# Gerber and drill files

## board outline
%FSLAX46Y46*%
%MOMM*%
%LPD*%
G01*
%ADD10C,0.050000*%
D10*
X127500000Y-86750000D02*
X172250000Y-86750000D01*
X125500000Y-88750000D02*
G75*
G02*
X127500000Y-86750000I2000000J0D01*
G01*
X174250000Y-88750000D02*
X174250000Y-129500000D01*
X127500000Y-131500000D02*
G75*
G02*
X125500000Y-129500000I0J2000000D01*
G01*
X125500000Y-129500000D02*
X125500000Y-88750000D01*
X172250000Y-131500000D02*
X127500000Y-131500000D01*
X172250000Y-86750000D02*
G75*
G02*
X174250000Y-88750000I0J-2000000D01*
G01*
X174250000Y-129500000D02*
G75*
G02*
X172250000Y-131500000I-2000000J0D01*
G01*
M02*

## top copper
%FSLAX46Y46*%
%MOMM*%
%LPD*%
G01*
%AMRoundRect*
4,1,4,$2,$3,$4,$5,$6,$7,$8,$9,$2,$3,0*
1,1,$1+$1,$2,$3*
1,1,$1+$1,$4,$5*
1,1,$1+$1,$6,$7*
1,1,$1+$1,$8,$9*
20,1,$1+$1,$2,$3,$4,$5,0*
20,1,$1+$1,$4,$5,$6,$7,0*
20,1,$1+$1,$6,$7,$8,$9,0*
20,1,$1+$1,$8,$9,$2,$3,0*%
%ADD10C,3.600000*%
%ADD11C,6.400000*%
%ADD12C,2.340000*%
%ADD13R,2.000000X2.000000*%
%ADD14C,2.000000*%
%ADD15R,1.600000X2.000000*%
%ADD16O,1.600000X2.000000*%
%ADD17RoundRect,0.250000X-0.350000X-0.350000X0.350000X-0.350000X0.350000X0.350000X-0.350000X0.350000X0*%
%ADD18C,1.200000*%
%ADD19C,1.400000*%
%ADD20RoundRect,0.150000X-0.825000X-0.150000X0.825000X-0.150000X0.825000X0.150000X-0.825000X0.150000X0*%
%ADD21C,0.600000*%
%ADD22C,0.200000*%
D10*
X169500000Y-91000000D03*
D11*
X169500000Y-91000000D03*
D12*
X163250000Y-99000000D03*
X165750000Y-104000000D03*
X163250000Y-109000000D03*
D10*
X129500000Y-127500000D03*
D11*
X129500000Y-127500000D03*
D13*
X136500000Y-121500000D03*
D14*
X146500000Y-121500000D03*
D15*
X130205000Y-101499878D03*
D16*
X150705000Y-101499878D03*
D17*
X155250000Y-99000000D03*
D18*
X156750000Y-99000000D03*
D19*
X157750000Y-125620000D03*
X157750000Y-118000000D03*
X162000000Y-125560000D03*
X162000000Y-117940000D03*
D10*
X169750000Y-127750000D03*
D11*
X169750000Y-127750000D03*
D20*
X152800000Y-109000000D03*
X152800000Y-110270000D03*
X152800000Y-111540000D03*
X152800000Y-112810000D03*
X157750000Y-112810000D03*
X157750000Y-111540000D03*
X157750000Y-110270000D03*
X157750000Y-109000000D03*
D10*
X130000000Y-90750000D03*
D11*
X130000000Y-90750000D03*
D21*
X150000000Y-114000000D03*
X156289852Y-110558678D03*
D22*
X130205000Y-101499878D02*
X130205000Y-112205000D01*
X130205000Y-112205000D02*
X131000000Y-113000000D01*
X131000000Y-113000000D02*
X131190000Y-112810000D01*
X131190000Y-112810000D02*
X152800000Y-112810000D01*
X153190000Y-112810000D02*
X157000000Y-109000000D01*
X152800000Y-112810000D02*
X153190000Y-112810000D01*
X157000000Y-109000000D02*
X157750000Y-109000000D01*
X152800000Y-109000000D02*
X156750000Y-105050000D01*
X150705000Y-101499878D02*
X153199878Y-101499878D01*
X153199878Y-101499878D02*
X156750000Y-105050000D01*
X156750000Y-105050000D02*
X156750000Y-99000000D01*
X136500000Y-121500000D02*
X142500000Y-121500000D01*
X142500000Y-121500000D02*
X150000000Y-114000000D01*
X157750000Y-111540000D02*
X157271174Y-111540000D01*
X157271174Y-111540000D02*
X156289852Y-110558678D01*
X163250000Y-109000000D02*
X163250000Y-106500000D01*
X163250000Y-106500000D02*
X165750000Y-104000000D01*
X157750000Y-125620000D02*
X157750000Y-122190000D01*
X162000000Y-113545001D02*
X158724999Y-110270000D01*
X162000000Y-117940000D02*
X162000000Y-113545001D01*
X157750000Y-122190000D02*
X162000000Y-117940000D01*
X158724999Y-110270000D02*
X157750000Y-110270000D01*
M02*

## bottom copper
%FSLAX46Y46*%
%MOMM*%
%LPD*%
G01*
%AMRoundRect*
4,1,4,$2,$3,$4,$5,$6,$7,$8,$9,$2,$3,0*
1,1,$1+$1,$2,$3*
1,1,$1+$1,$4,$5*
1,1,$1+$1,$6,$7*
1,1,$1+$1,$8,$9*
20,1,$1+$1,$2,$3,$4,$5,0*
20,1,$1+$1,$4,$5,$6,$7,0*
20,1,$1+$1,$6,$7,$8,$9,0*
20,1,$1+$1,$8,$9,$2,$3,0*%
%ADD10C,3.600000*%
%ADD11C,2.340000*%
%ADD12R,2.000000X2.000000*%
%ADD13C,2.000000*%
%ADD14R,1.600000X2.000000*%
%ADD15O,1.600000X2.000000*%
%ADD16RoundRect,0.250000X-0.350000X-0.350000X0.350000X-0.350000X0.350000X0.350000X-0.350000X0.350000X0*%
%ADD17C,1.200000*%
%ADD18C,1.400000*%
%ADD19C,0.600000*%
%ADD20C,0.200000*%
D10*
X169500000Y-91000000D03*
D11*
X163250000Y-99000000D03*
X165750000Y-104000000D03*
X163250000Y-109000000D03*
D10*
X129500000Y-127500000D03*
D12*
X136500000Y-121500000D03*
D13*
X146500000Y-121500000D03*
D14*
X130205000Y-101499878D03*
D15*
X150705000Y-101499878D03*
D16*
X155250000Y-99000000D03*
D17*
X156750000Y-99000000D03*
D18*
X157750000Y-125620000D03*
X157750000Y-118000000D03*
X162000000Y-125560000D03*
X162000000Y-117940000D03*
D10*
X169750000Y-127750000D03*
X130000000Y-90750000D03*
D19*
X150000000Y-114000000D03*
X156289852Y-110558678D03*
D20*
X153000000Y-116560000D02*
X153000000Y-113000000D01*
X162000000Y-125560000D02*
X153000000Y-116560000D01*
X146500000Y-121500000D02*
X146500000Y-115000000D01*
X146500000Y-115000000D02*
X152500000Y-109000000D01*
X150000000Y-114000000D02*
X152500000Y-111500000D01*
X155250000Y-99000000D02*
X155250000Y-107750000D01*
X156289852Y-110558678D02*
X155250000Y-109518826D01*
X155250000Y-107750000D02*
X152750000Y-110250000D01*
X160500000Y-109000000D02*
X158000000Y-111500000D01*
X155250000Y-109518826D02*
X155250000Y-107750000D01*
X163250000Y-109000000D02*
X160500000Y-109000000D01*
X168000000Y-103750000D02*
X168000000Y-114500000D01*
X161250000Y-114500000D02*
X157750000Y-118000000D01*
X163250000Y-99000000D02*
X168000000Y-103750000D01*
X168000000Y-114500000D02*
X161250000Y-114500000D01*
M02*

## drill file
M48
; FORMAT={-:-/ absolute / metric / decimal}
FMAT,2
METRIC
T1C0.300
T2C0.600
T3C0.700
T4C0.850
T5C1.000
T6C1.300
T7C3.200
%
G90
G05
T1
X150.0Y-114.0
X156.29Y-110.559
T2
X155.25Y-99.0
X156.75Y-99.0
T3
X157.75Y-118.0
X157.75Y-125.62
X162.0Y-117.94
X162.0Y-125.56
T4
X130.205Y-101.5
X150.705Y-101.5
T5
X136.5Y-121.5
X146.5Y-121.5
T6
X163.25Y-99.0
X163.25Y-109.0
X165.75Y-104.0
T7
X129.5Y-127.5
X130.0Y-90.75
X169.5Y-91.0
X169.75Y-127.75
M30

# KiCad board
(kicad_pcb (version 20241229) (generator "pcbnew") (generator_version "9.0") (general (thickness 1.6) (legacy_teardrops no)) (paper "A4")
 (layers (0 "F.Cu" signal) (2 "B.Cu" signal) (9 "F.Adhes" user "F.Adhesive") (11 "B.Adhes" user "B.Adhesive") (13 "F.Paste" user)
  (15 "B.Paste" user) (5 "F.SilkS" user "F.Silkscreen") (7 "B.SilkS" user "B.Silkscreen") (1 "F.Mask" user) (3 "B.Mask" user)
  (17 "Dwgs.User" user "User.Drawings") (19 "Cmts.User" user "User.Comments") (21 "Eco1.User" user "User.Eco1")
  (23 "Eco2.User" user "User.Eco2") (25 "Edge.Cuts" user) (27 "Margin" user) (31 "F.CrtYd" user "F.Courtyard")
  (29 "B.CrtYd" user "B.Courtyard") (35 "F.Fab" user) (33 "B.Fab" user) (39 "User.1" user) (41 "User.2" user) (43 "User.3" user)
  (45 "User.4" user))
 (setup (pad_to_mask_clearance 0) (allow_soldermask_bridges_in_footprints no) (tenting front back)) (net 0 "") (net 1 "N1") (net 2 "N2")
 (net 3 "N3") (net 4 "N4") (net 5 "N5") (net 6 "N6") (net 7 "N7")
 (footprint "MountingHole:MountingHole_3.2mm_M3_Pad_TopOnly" (layer "F.Cu") (at 169.5 91)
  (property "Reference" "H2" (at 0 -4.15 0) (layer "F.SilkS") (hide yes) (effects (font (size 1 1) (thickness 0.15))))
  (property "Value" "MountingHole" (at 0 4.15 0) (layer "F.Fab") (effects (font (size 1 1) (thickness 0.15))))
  (pad "1" thru_hole circle (at 0 0) (size 3.6 3.6) (drill 3.2) (layers "*.Cu" "*.Mask") (remove_unused_layers no) (zone_connect 2))
  (pad "1" connect circle (at 0 0) (size 6.4 6.4) (layers "F.Cu" "F.Mask") (zone_connect 2)))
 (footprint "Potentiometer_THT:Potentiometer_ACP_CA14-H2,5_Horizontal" (layer "F.Cu") (at 163.25 99)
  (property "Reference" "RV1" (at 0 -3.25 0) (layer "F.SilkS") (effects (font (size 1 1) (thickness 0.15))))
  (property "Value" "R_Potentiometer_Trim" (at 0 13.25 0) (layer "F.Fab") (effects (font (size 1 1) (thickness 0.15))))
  (pad "1" thru_hole circle (at 0 0) (size 2.34 2.34) (drill 1.3) (layers "*.Cu" "*.Mask") (remove_unused_layers no) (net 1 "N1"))
  (pad "2" thru_hole circle (at 2.5 5) (size 2.34 2.34) (drill 1.3) (layers "*.Cu" "*.Mask") (remove_unused_layers no) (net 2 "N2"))
  (pad "3" thru_hole circle (at 0 10) (size 2.34 2.34) (drill 1.3) (layers "*.Cu" "*.Mask") (remove_unused_layers no) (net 2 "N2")))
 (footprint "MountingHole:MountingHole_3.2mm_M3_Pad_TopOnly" (layer "F.Cu") (at 129.5 127.5)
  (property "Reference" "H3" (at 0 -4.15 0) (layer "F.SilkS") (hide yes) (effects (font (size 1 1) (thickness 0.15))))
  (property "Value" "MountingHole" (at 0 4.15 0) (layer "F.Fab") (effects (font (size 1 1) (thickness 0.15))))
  (pad "1" thru_hole circle (at 0 0) (size 3.6 3.6) (drill 3.2) (layers "*.Cu" "*.Mask") (remove_unused_layers no) (zone_connect 2))
  (pad "1" connect circle (at 0 0) (size 6.4 6.4) (layers "F.Cu" "F.Mask") (zone_connect 2)))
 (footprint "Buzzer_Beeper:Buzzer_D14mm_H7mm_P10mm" (layer "F.Cu") (at 136.5 121.5)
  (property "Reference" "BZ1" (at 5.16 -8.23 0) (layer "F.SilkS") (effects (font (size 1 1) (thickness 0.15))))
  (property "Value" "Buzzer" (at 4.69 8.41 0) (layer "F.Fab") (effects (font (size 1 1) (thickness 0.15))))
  (pad "1" thru_hole rect (at 0 0) (size 2 2) (drill 1) (layers "*.Cu" "*.Mask") (remove_unused_layers no) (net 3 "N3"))
  (pad "2" thru_hole circle (at 10 0) (size 2 2) (drill 1) (layers "*.Cu" "*.Mask") (remove_unused_layers no) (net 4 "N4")))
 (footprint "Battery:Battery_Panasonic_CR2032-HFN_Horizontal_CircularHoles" (layer "F.Cu") (at 130.205 101.499878)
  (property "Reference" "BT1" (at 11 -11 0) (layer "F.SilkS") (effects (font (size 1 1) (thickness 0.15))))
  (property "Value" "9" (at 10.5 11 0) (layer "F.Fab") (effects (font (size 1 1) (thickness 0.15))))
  (pad "1" thru_hole rect (at 0 0) (size 1.6 2) (drill 0.85) (layers "*.Cu" "*.Mask") (remove_unused_layers no) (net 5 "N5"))
  (pad "2" thru_hole oval (at 20.5 0) (size 1.6 2) (drill 0.85) (layers "*.Cu" "*.Mask") (remove_unused_layers no) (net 4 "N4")))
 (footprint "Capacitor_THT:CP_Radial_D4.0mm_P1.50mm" (layer "F.Cu") (at 155.25 99)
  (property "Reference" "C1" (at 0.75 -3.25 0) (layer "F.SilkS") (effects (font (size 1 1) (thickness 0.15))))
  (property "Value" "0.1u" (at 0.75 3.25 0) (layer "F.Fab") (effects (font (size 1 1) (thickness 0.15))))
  (pad "1" thru_hole roundrect (at 0 0) (size 1.2 1.2) (drill 0.6) (layers "*.Cu" "*.Mask") (remove_unused_layers no)
   (roundrect_rratio 0.208333) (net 2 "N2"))
  (pad "2" thru_hole circle (at 1.5 0) (size 1.2 1.2) (drill 0.6) (layers "*.Cu" "*.Mask") (remove_unused_layers no) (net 4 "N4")))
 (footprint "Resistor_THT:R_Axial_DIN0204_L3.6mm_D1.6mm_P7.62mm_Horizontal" (layer "F.Cu") (at 157.75 125.62 90)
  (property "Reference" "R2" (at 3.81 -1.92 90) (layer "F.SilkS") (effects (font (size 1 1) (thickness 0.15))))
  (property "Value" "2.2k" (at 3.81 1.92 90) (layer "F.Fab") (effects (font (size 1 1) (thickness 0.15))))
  (pad "1" thru_hole circle (at 0 0 90) (size 1.4 1.4) (drill 0.7) (layers "*.Cu" "*.Mask") (remove_unused_layers no) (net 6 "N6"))
  (pad "2" thru_hole circle (at 7.62 0 90) (size 1.4 1.4) (drill 0.7) (layers "*.Cu" "*.Mask") (remove_unused_layers no) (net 1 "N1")))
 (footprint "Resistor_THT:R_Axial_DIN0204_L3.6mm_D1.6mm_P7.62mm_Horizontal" (layer "F.Cu") (at 162 125.56 90)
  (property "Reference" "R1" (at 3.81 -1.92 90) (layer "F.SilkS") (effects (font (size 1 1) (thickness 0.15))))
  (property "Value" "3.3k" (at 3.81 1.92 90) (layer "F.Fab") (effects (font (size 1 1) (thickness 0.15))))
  (pad "1" thru_hole circle (at 0 0 90) (size 1.4 1.4) (drill 0.7) (layers "*.Cu" "*.Mask") (remove_unused_layers no) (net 5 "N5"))
  (pad "2" thru_hole circle (at 7.62 0 90) (size 1.4 1.4) (drill 0.7) (layers "*.Cu" "*.Mask") (remove_unused_layers no) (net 6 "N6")))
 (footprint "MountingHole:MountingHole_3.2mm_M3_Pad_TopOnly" (layer "F.Cu") (at 169.75 127.75)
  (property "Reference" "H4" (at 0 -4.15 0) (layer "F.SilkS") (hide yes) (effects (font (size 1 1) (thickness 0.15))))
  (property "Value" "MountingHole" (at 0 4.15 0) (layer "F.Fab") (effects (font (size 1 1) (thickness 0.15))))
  (pad "1" thru_hole circle (at 0 0) (size 3.6 3.6) (drill 3.2) (layers "*.Cu" "*.Mask") (remove_unused_layers no) (zone_connect 2))
  (pad "1" connect circle (at 0 0) (size 6.4 6.4) (layers "F.Cu" "F.Mask") (zone_connect 2)))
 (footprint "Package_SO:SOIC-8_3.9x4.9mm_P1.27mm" (layer "F.Cu") (at 155.275 110.905)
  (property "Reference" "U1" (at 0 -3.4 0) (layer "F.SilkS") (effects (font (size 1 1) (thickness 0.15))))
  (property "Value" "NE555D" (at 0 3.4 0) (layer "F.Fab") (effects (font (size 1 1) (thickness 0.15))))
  (pad "1" smd roundrect (at -2.475 -1.905) (size 1.95 0.6) (layers "F.Cu" "F.Mask" "F.Paste") (roundrect_rratio 0.25) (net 4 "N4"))
  (pad "2" smd roundrect (at -2.475 -0.635) (size 1.95 0.6) (layers "F.Cu" "F.Mask" "F.Paste") (roundrect_rratio 0.25) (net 2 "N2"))
  (pad "3" smd roundrect (at -2.475 0.635) (size 1.95 0.6) (layers "F.Cu" "F.Mask" "F.Paste") (roundrect_rratio 0.25) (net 3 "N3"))
  (pad "4" smd roundrect (at -2.475 1.905) (size 1.95 0.6) (layers "F.Cu" "F.Mask" "F.Paste") (roundrect_rratio 0.25) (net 5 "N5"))
  (pad "5" smd roundrect (at 2.475 1.905) (size 1.95 0.6) (layers "F.Cu" "F.Mask" "F.Paste") (roundrect_rratio 0.25) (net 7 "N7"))
  (pad "6" smd roundrect (at 2.475 0.635) (size 1.95 0.6) (layers "F.Cu" "F.Mask" "F.Paste") (roundrect_rratio 0.25) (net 2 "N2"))
  (pad "7" smd roundrect (at 2.475 -0.635) (size 1.95 0.6) (layers "F.Cu" "F.Mask" "F.Paste") (roundrect_rratio 0.25) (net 6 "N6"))
  (pad "8" smd roundrect (at 2.475 -1.905) (size 1.95 0.6) (layers "F.Cu" "F.Mask" "F.Paste") (roundrect_rratio 0.25) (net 5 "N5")))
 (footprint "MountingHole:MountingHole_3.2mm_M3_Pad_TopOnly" (layer "F.Cu") (at 130 90.75)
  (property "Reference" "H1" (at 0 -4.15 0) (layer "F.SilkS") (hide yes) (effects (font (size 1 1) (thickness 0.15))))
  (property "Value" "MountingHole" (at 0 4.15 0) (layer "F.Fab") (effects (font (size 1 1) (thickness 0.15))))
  (pad "1" thru_hole circle (at 0 0) (size 3.6 3.6) (drill 3.2) (layers "*.Cu" "*.Mask") (remove_unused_layers no) (zone_connect 2))
  (pad "1" connect circle (at 0 0) (size 6.4 6.4) (layers "F.Cu" "F.Mask") (zone_connect 2)))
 (gr_line (start 127.5 86.75) (end 172.25 86.75) (stroke (width 0.05) (type default)) (layer "Edge.Cuts"))
 (gr_arc (start 125.5 88.75) (mid 126.085786 87.335786) (end 127.5 86.75) (stroke (width 0.05) (type default)) (layer "Edge.Cuts"))
 (gr_line (start 174.25 88.75) (end 174.25 129.5) (stroke (width 0.05) (type default)) (layer "Edge.Cuts"))
 (gr_arc (start 127.5 131.5) (mid 126.085786 130.914214) (end 125.5 129.5) (stroke (width 0.05) (type default)) (layer "Edge.Cuts"))
 (gr_line (start 125.5 129.5) (end 125.5 88.75) (stroke (width 0.05) (type default)) (layer "Edge.Cuts"))
 (gr_line (start 172.25 131.5) (end 127.5 131.5) (stroke (width 0.05) (type default)) (layer "Edge.Cuts"))
 (gr_arc (start 172.25 86.75) (mid 173.664214 87.335786) (end 174.25 88.75) (stroke (width 0.05) (type default)) (layer "Edge.Cuts"))
 (gr_arc (start 174.25 129.5) (mid 173.664214 130.914214) (end 172.25 131.5) (stroke (width 0.05) (type default)) (layer "Edge.Cuts"))
 (segment (start 130.205 101.499878) (end 130.205 112.205) (width 0.2) (layer "F.Cu") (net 5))
 (segment (start 130.205 112.205) (end 131 113) (width 0.2) (layer "F.Cu") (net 5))
 (segment (start 131 113) (end 131.19 112.81) (width 0.2) (layer "F.Cu") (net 5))
 (segment (start 131.19 112.81) (end 152.8 112.81) (width 0.2) (layer "F.Cu") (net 5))
 (segment (start 153.19 112.81) (end 157 109) (width 0.2) (layer "F.Cu") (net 5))
 (segment (start 152.8 112.81) (end 153.19 112.81) (width 0.2) (layer "F.Cu") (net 5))
 (segment (start 157 109) (end 157.75 109) (width 0.2) (layer "F.Cu") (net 5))
 (segment (start 153 116.56) (end 153 113) (width 0.2) (layer "B.Cu") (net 5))
 (segment (start 162 125.56) (end 153 116.56) (width 0.2) (layer "B.Cu") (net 5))
 (segment (start 152.8 109) (end 156.75 105.05) (width 0.2) (layer "F.Cu") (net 4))
 (segment (start 150.705 101.499878) (end 153.199878 101.499878) (width 0.2) (layer "F.Cu") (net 4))
 (segment (start 153.199878 101.499878) (end 156.75 105.05) (width 0.2) (layer "F.Cu") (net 4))
 (segment (start 156.75 105.05) (end 156.75 99) (width 0.2) (layer "F.Cu") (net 4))
 (segment (start 146.5 121.5) (end 146.5 115) (width 0.2) (layer "B.Cu") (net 4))
 (segment (start 146.5 115) (end 152.5 109) (width 0.2) (layer "B.Cu") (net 4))
 (segment (start 136.5 121.5) (end 142.5 121.5) (width 0.2) (layer "F.Cu") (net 3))
 (segment (start 142.5 121.5) (end 150 114) (width 0.2) (layer "F.Cu") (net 3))
 (via (at 150 114) (size 0.6) (drill 0.3) (layers "F.Cu" "B.Cu") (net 3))
 (segment (start 150 114) (end 152.5 111.5) (width 0.2) (layer "B.Cu") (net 3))
 (segment (start 157.75 111.54) (end 157.271174 111.54) (width 0.2) (layer "F.Cu") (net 2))
 (segment (start 157.271174 111.54) (end 156.289852 110.558678) (width 0.2) (layer "F.Cu") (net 2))
 (segment (start 163.25 109) (end 163.25 106.5) (width 0.2) (layer "F.Cu") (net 2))
 (segment (start 163.25 106.5) (end 165.75 104) (width 0.2) (layer "F.Cu") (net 2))
 (via (at 156.289852 110.558678) (size 0.6) (drill 0.3) (layers "F.Cu" "B.Cu") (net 2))
 (segment (start 155.25 99) (end 155.25 107.75) (width 0.2) (layer "B.Cu") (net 2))
 (segment (start 156.289852 110.558678) (end 155.25 109.518826) (width 0.2) (layer "B.Cu") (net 2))
 (segment (start 155.25 107.75) (end 152.75 110.25) (width 0.2) (layer "B.Cu") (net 2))
 (segment (start 160.5 109) (end 158 111.5) (width 0.2) (layer "B.Cu") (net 2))
 (segment (start 155.25 109.518826) (end 155.25 107.75) (width 0.2) (layer "B.Cu") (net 2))
 (segment (start 163.25 109) (end 160.5 109) (width 0.2) (layer "B.Cu") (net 2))
 (segment (start 157.75 125.62) (end 157.75 122.19) (width 0.2) (layer "F.Cu") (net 6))
 (segment (start 162 113.545001) (end 158.724999 110.27) (width 0.2) (layer "F.Cu") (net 6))
 (segment (start 162 117.94) (end 162 113.545001) (width 0.2) (layer "F.Cu") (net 6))
 (segment (start 157.75 122.19) (end 162 117.94) (width 0.2) (layer "F.Cu") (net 6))
 (segment (start 158.724999 110.27) (end 157.75 110.27) (width 0.2) (layer "F.Cu") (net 6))
 (segment (start 168 103.75) (end 168 114.5) (width 0.2) (layer "B.Cu") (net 1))
 (segment (start 161.25 114.5) (end 157.75 118) (width 0.2) (layer "B.Cu") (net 1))
 (segment (start 163.25 99) (end 168 103.75) (width 0.2) (layer "B.Cu") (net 1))
 (segment (start 168 114.5) (end 161.25 114.5) (width 0.2) (layer "B.Cu") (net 1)))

